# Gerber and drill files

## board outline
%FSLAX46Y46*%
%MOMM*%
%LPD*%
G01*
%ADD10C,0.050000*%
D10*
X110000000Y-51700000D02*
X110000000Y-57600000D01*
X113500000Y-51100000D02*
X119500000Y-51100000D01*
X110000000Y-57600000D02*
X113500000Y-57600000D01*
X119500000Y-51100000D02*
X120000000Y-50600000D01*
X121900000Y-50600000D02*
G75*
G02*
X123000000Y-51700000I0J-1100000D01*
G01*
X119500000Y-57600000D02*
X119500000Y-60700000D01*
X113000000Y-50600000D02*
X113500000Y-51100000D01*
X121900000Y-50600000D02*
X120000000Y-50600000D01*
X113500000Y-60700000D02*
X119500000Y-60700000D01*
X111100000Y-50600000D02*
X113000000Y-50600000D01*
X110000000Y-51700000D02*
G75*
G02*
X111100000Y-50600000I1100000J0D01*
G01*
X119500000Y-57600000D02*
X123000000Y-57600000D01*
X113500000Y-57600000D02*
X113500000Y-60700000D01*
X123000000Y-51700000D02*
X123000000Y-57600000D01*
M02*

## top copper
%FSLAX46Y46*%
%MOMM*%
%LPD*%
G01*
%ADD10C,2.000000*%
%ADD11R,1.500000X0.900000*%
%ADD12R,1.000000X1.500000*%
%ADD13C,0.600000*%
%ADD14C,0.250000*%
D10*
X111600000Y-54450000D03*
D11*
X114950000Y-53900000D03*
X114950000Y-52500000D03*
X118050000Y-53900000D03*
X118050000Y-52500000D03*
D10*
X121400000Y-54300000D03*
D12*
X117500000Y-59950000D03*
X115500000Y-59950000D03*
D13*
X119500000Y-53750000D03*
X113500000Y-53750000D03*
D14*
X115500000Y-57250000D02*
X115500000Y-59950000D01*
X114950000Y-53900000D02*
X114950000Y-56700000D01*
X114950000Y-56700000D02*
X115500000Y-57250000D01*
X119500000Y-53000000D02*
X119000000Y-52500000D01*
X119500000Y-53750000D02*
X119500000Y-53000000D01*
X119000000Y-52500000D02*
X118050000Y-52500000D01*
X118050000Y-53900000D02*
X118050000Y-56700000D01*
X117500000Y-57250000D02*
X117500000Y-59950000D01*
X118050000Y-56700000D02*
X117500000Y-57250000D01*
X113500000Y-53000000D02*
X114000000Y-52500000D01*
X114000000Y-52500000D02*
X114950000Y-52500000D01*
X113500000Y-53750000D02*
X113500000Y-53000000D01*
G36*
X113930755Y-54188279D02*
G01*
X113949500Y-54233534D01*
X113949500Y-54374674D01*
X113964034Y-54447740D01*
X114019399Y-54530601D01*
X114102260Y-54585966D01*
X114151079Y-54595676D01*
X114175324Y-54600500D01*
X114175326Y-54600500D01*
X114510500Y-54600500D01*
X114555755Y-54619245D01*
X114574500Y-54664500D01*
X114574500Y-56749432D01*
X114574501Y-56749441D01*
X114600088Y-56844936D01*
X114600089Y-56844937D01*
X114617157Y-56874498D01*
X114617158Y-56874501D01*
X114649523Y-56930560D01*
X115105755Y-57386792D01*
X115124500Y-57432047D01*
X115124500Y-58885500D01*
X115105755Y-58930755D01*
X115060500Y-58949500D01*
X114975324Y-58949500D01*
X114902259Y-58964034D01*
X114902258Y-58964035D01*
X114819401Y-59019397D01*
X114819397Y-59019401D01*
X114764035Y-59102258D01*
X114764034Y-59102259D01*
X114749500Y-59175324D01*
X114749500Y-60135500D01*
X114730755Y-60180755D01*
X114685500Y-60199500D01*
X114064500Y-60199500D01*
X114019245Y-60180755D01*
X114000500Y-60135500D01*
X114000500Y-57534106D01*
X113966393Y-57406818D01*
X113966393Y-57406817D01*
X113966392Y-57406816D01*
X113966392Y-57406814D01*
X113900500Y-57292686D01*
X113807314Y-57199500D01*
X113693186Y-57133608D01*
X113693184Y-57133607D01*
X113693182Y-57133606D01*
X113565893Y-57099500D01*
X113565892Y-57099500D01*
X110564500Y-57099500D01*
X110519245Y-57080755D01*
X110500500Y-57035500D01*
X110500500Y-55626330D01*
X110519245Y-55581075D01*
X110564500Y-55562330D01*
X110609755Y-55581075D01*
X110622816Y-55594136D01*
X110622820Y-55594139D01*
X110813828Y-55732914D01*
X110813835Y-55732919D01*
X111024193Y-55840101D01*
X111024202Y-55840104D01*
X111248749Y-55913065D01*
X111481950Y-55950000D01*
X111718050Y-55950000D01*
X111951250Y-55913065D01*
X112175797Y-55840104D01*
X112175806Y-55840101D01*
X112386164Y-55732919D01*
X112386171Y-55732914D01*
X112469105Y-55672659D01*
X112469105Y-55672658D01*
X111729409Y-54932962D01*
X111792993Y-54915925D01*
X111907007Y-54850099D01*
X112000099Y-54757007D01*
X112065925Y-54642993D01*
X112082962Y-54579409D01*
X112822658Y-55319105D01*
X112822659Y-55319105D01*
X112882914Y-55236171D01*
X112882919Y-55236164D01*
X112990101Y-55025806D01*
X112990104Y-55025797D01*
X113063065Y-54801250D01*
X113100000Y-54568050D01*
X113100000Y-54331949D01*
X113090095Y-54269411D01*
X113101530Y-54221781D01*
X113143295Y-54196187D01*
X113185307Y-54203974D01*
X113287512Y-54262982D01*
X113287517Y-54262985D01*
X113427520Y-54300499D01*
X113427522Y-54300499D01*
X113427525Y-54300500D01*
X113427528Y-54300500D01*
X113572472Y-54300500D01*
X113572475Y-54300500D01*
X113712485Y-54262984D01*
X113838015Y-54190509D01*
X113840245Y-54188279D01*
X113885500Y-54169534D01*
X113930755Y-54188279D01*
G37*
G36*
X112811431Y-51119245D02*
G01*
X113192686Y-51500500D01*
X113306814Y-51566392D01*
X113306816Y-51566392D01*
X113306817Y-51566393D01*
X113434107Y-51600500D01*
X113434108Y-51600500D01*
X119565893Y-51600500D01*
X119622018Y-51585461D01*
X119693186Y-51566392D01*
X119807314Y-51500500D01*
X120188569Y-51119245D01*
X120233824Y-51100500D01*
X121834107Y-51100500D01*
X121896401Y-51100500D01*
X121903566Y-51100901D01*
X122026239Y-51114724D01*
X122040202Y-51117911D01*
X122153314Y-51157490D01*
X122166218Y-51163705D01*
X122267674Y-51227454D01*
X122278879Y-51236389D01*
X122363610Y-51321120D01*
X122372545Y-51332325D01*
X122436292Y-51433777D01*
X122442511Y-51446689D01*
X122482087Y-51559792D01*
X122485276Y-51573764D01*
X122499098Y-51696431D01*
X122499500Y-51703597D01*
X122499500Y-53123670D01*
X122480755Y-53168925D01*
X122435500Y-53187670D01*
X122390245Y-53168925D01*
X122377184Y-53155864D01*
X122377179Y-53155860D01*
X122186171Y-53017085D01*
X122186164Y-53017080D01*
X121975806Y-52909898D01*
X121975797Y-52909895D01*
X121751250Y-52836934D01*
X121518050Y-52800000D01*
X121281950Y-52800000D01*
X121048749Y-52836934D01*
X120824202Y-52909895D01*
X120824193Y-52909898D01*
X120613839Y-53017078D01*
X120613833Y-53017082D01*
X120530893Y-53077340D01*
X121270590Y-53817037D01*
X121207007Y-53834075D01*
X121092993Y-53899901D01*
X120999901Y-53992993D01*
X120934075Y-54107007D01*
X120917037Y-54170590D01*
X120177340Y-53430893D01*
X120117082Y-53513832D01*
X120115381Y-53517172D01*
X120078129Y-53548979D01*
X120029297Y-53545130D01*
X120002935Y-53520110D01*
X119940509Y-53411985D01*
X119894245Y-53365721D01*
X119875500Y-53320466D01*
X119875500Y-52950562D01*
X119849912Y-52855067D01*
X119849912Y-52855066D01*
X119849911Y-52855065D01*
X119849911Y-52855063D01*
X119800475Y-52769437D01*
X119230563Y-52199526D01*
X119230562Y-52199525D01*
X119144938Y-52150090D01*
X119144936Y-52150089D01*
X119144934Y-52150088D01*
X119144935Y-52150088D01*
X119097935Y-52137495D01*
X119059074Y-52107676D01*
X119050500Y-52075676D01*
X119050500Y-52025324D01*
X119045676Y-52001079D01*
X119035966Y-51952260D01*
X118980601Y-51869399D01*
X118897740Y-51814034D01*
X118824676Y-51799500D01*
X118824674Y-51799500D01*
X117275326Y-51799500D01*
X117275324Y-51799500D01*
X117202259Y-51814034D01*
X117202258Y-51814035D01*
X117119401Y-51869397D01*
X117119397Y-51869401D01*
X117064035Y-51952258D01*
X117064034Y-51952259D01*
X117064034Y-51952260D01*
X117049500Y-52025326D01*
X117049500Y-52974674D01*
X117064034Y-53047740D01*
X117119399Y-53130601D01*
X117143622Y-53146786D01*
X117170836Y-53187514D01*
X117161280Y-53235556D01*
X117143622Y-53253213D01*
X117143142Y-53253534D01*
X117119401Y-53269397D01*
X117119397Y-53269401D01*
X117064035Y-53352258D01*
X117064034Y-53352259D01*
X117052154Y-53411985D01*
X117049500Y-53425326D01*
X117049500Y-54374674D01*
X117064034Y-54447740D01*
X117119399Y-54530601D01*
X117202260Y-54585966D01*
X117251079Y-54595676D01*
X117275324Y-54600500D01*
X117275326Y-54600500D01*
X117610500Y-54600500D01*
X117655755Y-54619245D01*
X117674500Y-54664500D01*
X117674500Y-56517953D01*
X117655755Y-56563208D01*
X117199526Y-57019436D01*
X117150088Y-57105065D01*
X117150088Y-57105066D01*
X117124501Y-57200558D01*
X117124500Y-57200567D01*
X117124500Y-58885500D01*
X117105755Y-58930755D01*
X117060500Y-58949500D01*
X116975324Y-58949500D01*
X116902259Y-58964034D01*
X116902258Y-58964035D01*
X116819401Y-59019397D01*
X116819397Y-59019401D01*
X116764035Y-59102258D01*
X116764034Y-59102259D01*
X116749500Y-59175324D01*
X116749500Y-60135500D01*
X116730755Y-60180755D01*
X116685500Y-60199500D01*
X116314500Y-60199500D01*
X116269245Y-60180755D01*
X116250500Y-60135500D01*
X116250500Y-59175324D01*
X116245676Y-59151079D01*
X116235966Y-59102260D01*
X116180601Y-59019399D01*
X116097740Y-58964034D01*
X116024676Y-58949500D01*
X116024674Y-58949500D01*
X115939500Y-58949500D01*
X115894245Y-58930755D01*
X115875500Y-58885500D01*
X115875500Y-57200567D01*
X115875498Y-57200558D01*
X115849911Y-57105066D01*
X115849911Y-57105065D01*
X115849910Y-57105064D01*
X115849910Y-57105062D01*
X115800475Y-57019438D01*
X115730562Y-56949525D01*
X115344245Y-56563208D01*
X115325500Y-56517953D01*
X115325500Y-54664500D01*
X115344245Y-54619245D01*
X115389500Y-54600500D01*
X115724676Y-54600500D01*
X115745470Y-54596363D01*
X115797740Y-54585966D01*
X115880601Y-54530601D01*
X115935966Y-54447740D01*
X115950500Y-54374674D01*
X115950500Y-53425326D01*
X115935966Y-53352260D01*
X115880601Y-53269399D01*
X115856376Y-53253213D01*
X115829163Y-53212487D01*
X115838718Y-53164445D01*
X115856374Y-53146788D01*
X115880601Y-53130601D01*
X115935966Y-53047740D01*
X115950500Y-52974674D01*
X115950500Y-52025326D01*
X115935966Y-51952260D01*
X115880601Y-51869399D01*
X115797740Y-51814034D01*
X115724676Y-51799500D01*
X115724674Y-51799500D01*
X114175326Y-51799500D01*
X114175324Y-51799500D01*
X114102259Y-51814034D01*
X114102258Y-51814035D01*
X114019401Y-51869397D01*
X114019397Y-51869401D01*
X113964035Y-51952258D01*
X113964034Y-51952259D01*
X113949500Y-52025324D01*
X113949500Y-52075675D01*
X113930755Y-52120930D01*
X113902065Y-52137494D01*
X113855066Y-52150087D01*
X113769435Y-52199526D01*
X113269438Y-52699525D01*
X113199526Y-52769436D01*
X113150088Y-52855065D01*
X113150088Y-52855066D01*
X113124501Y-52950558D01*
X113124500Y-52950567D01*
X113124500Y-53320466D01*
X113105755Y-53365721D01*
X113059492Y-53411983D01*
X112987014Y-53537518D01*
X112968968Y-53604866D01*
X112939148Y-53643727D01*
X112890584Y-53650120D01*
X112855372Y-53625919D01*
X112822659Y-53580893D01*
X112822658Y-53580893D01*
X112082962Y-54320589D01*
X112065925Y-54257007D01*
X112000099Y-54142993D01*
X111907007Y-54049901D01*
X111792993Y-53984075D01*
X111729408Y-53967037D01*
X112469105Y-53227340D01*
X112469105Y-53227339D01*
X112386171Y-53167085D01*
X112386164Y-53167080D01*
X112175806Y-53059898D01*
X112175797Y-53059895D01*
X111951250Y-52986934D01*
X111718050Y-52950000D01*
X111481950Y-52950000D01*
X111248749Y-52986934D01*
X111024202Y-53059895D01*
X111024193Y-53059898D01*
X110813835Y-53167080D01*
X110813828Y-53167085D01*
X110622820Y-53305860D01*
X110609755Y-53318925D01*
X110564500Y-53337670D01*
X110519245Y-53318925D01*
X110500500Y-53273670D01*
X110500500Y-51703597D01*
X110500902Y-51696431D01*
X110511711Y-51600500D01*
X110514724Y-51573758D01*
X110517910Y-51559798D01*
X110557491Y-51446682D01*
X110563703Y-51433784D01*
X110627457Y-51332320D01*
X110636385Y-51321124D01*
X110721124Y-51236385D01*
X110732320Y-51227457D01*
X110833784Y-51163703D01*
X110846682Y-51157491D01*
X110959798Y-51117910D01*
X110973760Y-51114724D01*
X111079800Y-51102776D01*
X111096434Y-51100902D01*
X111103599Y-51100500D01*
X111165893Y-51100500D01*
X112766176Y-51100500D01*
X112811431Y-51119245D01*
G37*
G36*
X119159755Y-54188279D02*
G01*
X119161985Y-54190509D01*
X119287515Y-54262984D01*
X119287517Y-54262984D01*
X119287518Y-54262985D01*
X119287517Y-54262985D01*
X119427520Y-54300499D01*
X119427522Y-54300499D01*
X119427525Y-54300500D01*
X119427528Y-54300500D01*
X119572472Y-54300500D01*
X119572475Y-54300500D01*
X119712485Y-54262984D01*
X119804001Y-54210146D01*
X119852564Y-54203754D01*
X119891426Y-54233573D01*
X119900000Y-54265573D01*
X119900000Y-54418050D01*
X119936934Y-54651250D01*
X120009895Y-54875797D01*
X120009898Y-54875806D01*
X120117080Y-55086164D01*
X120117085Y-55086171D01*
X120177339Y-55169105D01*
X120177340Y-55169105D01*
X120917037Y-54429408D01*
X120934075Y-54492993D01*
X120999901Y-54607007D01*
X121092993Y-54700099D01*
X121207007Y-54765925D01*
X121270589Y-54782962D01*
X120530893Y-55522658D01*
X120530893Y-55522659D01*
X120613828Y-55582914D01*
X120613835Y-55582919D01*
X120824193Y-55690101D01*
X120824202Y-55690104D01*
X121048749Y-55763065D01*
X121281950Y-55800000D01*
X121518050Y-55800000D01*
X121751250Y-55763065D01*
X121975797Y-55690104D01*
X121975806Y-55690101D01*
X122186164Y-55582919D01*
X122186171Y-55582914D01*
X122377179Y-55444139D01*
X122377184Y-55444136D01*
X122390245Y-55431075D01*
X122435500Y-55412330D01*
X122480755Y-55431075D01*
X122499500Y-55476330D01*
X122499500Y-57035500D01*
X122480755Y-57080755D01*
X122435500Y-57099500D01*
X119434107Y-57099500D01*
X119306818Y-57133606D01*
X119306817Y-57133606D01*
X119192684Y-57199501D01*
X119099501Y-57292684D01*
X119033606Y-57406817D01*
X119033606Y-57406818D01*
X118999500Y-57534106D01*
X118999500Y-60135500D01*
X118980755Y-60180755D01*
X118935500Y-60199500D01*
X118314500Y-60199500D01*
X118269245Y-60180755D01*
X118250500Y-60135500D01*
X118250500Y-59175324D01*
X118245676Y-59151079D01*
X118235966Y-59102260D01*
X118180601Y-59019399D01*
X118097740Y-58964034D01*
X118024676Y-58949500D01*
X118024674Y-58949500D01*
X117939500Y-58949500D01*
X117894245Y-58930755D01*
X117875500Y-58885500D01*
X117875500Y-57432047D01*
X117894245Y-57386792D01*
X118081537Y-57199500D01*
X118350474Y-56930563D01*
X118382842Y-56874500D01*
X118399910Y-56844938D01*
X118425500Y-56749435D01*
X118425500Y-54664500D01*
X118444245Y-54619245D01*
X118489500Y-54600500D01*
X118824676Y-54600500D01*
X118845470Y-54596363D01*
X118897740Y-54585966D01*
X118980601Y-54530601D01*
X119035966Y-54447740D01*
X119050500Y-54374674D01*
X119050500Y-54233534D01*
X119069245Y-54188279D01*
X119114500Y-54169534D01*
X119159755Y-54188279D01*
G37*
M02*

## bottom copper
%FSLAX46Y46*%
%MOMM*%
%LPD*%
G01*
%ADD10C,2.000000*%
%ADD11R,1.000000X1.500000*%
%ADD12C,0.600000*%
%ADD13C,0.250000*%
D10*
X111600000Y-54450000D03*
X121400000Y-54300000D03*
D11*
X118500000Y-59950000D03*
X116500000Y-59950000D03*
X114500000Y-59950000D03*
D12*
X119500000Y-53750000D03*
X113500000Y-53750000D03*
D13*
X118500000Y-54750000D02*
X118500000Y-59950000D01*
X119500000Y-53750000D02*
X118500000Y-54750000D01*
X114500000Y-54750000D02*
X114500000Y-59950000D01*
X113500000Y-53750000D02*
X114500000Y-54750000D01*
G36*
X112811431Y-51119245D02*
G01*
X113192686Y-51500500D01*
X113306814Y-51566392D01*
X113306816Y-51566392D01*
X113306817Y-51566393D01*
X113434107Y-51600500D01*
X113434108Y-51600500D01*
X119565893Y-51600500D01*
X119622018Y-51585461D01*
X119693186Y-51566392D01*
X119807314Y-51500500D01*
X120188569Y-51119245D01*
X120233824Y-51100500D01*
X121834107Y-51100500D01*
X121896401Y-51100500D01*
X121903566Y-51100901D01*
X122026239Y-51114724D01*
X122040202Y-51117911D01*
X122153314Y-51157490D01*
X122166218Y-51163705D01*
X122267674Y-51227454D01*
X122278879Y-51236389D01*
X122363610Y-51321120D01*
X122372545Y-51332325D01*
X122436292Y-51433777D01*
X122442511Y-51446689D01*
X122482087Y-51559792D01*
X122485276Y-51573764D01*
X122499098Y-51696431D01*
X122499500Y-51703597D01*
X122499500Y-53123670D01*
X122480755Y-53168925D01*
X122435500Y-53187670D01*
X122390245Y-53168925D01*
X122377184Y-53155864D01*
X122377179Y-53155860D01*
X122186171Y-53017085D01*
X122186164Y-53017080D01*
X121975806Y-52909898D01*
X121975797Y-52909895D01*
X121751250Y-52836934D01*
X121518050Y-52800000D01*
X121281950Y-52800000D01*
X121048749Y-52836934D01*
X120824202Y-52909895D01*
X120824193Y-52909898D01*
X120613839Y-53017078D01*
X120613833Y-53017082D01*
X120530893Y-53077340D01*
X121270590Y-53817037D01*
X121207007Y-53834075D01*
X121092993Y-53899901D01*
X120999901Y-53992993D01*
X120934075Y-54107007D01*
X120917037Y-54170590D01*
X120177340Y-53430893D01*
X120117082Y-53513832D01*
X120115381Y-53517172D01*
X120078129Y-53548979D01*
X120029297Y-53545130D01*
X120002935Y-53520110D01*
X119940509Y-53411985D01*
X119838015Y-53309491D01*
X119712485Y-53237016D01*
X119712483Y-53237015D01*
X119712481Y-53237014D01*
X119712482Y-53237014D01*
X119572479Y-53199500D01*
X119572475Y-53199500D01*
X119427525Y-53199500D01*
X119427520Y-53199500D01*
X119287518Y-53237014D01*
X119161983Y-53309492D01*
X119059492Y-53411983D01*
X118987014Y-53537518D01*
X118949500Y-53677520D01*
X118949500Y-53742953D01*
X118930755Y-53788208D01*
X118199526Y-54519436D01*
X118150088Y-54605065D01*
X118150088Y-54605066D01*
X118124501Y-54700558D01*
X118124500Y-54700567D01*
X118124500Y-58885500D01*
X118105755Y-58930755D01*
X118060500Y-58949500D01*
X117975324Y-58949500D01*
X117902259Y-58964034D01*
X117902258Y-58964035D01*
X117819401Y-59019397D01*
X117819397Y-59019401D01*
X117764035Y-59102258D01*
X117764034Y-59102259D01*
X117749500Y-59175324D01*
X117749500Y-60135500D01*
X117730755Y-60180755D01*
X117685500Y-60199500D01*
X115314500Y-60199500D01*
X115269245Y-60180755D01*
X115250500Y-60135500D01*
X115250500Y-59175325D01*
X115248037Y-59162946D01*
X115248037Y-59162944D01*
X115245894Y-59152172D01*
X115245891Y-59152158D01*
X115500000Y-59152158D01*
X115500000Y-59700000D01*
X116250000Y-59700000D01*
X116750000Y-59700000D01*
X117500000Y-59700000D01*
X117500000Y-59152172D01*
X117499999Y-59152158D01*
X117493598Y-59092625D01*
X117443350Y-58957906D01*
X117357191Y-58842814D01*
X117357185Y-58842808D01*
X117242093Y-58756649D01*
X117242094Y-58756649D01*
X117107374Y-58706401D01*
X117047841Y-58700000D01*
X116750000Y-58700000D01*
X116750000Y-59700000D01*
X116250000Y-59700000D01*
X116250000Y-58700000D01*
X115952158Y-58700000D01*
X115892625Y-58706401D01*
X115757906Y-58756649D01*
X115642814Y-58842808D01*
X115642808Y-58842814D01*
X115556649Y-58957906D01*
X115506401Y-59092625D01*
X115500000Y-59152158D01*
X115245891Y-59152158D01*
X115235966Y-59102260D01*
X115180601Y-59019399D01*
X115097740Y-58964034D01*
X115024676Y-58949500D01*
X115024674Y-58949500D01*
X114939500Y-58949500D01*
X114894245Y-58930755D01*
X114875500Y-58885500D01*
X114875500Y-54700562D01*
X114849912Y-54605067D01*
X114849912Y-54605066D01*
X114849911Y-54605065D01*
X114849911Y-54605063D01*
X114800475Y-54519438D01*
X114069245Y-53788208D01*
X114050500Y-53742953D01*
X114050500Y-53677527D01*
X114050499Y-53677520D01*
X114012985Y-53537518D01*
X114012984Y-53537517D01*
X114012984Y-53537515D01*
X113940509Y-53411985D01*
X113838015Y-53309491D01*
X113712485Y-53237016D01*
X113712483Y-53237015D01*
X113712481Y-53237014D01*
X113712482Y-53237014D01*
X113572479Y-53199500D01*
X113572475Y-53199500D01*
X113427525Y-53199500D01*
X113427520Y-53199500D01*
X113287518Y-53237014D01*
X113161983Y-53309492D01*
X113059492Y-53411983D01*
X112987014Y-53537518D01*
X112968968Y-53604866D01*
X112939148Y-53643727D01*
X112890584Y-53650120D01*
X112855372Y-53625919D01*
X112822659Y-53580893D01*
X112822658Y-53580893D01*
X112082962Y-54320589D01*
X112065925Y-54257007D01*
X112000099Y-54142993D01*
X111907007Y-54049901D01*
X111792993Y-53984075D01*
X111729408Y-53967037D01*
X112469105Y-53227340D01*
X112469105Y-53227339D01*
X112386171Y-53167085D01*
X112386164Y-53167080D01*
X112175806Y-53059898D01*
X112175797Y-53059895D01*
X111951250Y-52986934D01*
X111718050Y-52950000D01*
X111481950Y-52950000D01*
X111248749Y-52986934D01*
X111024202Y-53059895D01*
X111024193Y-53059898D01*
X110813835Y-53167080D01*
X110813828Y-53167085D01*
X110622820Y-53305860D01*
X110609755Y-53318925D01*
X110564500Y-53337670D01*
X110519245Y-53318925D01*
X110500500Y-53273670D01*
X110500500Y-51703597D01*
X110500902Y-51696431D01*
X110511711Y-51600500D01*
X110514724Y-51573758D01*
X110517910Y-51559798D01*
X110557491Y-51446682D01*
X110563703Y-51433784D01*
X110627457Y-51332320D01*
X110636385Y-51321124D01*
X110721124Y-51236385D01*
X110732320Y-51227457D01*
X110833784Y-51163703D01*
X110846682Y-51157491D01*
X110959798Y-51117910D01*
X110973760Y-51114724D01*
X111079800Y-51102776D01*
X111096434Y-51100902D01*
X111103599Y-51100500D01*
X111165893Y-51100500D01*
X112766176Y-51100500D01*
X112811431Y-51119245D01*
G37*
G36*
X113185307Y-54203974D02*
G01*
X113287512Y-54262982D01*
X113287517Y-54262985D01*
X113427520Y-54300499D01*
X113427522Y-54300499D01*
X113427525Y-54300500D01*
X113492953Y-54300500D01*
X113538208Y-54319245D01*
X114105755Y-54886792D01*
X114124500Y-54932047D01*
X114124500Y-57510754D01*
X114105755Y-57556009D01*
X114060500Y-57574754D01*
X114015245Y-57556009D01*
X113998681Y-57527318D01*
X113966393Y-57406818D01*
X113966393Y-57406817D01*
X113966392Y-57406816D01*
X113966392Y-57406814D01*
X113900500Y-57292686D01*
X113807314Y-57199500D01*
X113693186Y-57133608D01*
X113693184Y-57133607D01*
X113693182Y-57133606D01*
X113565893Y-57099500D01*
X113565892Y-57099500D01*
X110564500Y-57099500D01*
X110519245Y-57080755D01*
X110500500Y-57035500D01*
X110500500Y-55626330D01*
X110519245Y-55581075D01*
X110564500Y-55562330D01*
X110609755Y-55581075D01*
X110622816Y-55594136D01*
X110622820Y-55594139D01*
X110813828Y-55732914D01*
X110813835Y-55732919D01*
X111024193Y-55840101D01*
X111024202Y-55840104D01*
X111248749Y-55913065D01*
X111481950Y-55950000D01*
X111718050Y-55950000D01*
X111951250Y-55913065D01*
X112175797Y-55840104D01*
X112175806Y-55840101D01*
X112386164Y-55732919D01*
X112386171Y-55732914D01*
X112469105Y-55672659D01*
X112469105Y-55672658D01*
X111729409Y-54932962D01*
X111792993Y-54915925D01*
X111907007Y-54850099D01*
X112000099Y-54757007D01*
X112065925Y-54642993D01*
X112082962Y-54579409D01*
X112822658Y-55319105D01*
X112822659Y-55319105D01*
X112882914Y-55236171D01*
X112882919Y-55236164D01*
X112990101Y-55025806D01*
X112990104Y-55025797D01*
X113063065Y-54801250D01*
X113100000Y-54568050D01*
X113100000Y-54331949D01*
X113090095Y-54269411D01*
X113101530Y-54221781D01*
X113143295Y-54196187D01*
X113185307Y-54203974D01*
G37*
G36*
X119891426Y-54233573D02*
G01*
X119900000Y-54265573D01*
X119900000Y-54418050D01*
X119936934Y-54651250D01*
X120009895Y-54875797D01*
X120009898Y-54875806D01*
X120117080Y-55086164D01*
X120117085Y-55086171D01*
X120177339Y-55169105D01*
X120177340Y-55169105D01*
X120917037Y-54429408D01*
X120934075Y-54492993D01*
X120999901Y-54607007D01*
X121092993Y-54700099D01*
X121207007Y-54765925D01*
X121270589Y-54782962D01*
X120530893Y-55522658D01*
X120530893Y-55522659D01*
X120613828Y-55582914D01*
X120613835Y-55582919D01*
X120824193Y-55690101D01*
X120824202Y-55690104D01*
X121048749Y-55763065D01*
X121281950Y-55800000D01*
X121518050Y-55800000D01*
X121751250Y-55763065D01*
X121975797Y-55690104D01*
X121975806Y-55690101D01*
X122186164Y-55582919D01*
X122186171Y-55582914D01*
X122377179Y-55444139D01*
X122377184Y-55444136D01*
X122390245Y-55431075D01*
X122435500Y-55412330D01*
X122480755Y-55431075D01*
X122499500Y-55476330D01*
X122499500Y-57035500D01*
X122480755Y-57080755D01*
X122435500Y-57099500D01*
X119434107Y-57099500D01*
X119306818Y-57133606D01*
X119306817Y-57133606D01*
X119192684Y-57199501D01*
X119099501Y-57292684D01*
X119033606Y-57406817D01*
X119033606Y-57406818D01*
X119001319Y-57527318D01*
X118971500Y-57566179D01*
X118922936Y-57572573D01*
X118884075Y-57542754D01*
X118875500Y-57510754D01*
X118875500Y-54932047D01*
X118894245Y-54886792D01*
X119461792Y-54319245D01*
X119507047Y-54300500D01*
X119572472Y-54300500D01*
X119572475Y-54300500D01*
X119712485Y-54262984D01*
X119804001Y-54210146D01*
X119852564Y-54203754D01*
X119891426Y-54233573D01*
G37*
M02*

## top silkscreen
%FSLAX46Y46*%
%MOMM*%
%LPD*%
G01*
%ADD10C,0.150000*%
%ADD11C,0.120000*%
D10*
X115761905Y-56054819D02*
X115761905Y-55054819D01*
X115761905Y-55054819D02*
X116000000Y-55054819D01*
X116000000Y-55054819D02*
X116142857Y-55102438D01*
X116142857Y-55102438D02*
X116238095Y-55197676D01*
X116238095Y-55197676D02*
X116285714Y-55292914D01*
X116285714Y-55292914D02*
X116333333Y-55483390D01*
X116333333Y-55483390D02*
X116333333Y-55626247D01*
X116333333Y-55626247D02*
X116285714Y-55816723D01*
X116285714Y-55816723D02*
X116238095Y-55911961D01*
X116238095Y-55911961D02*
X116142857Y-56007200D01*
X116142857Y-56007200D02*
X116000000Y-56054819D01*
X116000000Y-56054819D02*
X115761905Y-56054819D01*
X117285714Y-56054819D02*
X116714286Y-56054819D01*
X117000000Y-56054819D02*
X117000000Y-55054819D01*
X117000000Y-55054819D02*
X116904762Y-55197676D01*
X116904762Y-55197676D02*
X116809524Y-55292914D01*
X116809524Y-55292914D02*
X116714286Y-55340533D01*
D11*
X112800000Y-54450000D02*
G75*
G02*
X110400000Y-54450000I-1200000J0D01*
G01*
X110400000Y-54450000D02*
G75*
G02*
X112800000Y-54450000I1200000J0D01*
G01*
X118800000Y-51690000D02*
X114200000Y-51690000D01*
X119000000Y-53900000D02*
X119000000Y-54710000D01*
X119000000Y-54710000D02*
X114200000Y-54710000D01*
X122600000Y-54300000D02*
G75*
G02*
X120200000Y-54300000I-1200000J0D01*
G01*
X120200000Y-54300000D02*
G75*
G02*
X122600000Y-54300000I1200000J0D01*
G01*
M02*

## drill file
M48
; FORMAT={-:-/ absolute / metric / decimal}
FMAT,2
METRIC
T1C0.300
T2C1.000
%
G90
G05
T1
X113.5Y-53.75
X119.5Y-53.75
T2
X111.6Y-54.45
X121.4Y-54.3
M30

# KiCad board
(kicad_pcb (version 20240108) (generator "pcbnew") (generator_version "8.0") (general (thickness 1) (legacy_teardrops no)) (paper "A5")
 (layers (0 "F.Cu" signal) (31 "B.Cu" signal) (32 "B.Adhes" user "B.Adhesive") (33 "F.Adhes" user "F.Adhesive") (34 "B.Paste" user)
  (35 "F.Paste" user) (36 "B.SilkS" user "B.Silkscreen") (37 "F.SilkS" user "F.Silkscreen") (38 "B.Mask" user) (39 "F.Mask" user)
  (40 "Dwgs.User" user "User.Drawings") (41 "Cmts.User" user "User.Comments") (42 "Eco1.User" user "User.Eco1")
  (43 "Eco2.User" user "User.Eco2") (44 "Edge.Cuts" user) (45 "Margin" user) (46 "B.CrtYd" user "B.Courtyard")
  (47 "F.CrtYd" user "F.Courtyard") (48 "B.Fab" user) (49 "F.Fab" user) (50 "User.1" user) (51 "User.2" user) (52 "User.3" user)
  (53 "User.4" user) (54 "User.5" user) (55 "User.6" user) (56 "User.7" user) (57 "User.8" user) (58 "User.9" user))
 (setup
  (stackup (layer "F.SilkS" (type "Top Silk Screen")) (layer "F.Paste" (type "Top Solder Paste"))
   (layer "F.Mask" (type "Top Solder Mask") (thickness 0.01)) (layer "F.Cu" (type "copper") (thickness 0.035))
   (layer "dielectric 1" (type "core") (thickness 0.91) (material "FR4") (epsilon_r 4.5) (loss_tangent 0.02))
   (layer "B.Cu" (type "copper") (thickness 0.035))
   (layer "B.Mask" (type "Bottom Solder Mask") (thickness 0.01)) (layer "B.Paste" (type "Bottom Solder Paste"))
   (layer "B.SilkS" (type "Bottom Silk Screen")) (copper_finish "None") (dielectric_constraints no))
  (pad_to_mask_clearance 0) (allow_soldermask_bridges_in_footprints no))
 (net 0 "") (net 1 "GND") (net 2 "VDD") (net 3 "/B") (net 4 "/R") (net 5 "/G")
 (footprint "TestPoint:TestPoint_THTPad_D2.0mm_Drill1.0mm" (layer "F.Cu") (at 111.6 54.45)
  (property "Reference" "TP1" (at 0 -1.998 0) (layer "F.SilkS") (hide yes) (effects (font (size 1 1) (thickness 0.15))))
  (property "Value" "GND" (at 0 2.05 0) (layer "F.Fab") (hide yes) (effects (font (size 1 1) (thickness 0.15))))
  (fp_circle (center 0 0) (end 0 1.2) (stroke (width 0.12) (type solid)) (fill none) (layer "F.SilkS"))
  (pad "1" thru_hole circle (at 0 0) (size 2 2) (drill 1) (layers "*.Cu" "*.Mask") (remove_unused_layers no) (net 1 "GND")))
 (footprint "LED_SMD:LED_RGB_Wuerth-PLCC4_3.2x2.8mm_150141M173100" (layer "F.Cu") (at 116.5 53.2 180)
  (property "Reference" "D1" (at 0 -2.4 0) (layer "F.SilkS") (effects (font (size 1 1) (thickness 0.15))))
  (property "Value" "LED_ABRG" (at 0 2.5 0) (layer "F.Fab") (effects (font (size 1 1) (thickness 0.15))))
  (fp_line (start -2.3 1.51) (end 2.3 1.51) (stroke (width 0.12) (type solid)) (layer "F.SilkS"))
  (fp_line (start -2.5 -0.7) (end -2.5 -1.51) (stroke (width 0.12) (type solid)) (layer "F.SilkS"))
  (fp_line (start -2.5 -1.51) (end 2.3 -1.51) (stroke (width 0.12) (type solid)) (layer "F.SilkS"))
  (pad "1" smd rect (at 1.55 -0.7 180) (size 1.5 0.9) (layers "F.Cu" "F.Paste" "F.Mask") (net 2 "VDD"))
  (pad "2" smd rect (at 1.55 0.7 180) (size 1.5 0.9) (layers "F.Cu" "F.Paste" "F.Mask") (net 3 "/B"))
  (pad "3" smd rect (at -1.55 -0.7 180) (size 1.5 0.9) (layers "F.Cu" "F.Paste" "F.Mask") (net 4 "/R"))
  (pad "4" smd rect (at -1.55 0.7 180) (size 1.5 0.9) (layers "F.Cu" "F.Paste" "F.Mask") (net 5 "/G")))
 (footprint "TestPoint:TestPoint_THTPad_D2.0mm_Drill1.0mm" (layer "F.Cu") (at 121.4 54.3)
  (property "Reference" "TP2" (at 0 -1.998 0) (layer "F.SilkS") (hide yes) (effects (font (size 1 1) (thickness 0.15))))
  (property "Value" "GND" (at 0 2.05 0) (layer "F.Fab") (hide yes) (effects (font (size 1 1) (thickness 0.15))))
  (fp_circle (center 0 0) (end 0 1.2) (stroke (width 0.12) (type solid)) (fill none) (layer "F.SilkS"))
  (pad "1" thru_hole circle (at 0 0) (size 2 2) (drill 1) (layers "*.Cu" "*.Mask") (remove_unused_layers no) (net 1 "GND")))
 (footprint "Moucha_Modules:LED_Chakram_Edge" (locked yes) (layer "B.Cu") (at 116.5 59.95 90)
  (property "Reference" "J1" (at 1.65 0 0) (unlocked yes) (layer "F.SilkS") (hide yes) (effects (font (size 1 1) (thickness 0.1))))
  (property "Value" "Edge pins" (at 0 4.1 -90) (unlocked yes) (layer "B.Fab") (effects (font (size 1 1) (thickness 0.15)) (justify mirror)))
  (pad "1" connect rect (at 0 2 90) (size 1.5 1) (layers "B.Cu" "B.Mask") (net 5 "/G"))
  (pad "2" connect rect (at 0 0 90) (size 1.5 1) (layers "B.Cu" "B.Mask") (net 1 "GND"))
  (pad "3" connect rect (at 0 -2 90) (size 1.5 1) (layers "B.Cu" "B.Mask") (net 3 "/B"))
  (pad "4" connect rect (at 0 1 90) (size 1.5 1) (layers "F.Cu" "F.Mask") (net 4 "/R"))
  (pad "5" connect rect (at 0 -1 90) (size 1.5 1) (layers "F.Cu" "F.Mask") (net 2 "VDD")))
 (gr_line (start 110 51.7) (end 110 57.6) (locked yes) (stroke (width 0.05) (type default)) (layer "Edge.Cuts"))
 (gr_line (start 113.5 51.1) (end 119.5 51.1) (locked yes) (stroke (width 0.05) (type default)) (layer "Edge.Cuts"))
 (gr_line (start 110 57.6) (end 113.5 57.6) (locked yes) (stroke (width 0.05) (type default)) (layer "Edge.Cuts"))
 (gr_line (start 119.5 51.1) (end 120 50.6) (locked yes) (stroke (width 0.05) (type default)) (layer "Edge.Cuts"))
 (gr_arc (start 121.9 50.6) (mid 122.677817 50.922183) (end 123 51.7) (locked yes) (stroke (width 0.05) (type default)) (layer "Edge.Cuts"))
 (gr_line (start 119.5 57.6) (end 119.5 60.7) (locked yes) (stroke (width 0.05) (type default)) (layer "Edge.Cuts"))
 (gr_line (start 113 50.6) (end 113.5 51.1) (locked yes) (stroke (width 0.05) (type default)) (layer "Edge.Cuts"))
 (gr_line (start 121.9 50.6) (end 120 50.6) (locked yes) (stroke (width 0.05) (type default)) (layer "Edge.Cuts"))
 (gr_line (start 113.5 60.7) (end 119.5 60.7) (locked yes) (stroke (width 0.05) (type default)) (layer "Edge.Cuts"))
 (gr_line (start 111.1 50.6) (end 113 50.6) (locked yes) (stroke (width 0.05) (type default)) (layer "Edge.Cuts"))
 (gr_arc (start 110 51.7) (mid 110.322183 50.922183) (end 111.1 50.6) (locked yes) (stroke (width 0.05) (type default)) (layer "Edge.Cuts"))
 (gr_line (start 119.5 57.6) (end 123 57.6) (locked yes) (stroke (width 0.05) (type default)) (layer "Edge.Cuts"))
 (gr_line (start 113.5 57.6) (end 113.5 60.7) (locked yes) (stroke (width 0.05) (type default)) (layer "Edge.Cuts"))
 (gr_line (start 123 51.7) (end 123 57.6) (locked yes) (stroke (width 0.05) (type default)) (layer "Edge.Cuts"))
 (segment (start 115.5 57.25) (end 115.5 59.95) (width 0.25) (layer "F.Cu") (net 2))
 (segment (start 114.95 53.9) (end 114.95 56.7) (width 0.25) (layer "F.Cu") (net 2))
 (segment (start 114.95 56.7) (end 115.5 57.25) (width 0.25) (layer "F.Cu") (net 2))
 (segment (start 119.5 53) (end 119 52.5) (width 0.25) (layer "F.Cu") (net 5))
 (segment (start 119.5 53.75) (end 119.5 53) (width 0.25) (layer "F.Cu") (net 5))
 (segment (start 119 52.5) (end 118.05 52.5) (width 0.25) (layer "F.Cu") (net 5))
 (via (at 119.5 53.75) (size 0.6) (drill 0.3) (layers "F.Cu" "B.Cu") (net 5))
 (segment (start 118.5 54.75) (end 118.5 59.95) (width 0.25) (layer "B.Cu") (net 5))
 (segment (start 119.5 53.75) (end 118.5 54.75) (width 0.25) (layer "B.Cu") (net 5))
 (segment (start 118.05 53.9) (end 118.05 56.7) (width 0.25) (layer "F.Cu") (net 4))
 (segment (start 117.5 57.25) (end 117.5 59.95) (width 0.25) (layer "F.Cu") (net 4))
 (segment (start 118.05 56.7) (end 117.5 57.25) (width 0.25) (layer "F.Cu") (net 4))
 (segment (start 113.5 53) (end 114 52.5) (width 0.25) (layer "F.Cu") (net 3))
 (segment (start 114 52.5) (end 114.95 52.5) (width 0.25) (layer "F.Cu") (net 3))
 (segment (start 113.5 53.75) (end 113.5 53) (width 0.25) (layer "F.Cu") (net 3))
 (via (at 113.5 53.75) (size 0.6) (drill 0.3) (layers "F.Cu" "B.Cu") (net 3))
 (segment (start 114.5 54.75) (end 114.5 59.95) (width 0.25) (layer "B.Cu") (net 3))
 (segment (start 113.5 53.75) (end 114.5 54.75) (width 0.25) (layer "B.Cu") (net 3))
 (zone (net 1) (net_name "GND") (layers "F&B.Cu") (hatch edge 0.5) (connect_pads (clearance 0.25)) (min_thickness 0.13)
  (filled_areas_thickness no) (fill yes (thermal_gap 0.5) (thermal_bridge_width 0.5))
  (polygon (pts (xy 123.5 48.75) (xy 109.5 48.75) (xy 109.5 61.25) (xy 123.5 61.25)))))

